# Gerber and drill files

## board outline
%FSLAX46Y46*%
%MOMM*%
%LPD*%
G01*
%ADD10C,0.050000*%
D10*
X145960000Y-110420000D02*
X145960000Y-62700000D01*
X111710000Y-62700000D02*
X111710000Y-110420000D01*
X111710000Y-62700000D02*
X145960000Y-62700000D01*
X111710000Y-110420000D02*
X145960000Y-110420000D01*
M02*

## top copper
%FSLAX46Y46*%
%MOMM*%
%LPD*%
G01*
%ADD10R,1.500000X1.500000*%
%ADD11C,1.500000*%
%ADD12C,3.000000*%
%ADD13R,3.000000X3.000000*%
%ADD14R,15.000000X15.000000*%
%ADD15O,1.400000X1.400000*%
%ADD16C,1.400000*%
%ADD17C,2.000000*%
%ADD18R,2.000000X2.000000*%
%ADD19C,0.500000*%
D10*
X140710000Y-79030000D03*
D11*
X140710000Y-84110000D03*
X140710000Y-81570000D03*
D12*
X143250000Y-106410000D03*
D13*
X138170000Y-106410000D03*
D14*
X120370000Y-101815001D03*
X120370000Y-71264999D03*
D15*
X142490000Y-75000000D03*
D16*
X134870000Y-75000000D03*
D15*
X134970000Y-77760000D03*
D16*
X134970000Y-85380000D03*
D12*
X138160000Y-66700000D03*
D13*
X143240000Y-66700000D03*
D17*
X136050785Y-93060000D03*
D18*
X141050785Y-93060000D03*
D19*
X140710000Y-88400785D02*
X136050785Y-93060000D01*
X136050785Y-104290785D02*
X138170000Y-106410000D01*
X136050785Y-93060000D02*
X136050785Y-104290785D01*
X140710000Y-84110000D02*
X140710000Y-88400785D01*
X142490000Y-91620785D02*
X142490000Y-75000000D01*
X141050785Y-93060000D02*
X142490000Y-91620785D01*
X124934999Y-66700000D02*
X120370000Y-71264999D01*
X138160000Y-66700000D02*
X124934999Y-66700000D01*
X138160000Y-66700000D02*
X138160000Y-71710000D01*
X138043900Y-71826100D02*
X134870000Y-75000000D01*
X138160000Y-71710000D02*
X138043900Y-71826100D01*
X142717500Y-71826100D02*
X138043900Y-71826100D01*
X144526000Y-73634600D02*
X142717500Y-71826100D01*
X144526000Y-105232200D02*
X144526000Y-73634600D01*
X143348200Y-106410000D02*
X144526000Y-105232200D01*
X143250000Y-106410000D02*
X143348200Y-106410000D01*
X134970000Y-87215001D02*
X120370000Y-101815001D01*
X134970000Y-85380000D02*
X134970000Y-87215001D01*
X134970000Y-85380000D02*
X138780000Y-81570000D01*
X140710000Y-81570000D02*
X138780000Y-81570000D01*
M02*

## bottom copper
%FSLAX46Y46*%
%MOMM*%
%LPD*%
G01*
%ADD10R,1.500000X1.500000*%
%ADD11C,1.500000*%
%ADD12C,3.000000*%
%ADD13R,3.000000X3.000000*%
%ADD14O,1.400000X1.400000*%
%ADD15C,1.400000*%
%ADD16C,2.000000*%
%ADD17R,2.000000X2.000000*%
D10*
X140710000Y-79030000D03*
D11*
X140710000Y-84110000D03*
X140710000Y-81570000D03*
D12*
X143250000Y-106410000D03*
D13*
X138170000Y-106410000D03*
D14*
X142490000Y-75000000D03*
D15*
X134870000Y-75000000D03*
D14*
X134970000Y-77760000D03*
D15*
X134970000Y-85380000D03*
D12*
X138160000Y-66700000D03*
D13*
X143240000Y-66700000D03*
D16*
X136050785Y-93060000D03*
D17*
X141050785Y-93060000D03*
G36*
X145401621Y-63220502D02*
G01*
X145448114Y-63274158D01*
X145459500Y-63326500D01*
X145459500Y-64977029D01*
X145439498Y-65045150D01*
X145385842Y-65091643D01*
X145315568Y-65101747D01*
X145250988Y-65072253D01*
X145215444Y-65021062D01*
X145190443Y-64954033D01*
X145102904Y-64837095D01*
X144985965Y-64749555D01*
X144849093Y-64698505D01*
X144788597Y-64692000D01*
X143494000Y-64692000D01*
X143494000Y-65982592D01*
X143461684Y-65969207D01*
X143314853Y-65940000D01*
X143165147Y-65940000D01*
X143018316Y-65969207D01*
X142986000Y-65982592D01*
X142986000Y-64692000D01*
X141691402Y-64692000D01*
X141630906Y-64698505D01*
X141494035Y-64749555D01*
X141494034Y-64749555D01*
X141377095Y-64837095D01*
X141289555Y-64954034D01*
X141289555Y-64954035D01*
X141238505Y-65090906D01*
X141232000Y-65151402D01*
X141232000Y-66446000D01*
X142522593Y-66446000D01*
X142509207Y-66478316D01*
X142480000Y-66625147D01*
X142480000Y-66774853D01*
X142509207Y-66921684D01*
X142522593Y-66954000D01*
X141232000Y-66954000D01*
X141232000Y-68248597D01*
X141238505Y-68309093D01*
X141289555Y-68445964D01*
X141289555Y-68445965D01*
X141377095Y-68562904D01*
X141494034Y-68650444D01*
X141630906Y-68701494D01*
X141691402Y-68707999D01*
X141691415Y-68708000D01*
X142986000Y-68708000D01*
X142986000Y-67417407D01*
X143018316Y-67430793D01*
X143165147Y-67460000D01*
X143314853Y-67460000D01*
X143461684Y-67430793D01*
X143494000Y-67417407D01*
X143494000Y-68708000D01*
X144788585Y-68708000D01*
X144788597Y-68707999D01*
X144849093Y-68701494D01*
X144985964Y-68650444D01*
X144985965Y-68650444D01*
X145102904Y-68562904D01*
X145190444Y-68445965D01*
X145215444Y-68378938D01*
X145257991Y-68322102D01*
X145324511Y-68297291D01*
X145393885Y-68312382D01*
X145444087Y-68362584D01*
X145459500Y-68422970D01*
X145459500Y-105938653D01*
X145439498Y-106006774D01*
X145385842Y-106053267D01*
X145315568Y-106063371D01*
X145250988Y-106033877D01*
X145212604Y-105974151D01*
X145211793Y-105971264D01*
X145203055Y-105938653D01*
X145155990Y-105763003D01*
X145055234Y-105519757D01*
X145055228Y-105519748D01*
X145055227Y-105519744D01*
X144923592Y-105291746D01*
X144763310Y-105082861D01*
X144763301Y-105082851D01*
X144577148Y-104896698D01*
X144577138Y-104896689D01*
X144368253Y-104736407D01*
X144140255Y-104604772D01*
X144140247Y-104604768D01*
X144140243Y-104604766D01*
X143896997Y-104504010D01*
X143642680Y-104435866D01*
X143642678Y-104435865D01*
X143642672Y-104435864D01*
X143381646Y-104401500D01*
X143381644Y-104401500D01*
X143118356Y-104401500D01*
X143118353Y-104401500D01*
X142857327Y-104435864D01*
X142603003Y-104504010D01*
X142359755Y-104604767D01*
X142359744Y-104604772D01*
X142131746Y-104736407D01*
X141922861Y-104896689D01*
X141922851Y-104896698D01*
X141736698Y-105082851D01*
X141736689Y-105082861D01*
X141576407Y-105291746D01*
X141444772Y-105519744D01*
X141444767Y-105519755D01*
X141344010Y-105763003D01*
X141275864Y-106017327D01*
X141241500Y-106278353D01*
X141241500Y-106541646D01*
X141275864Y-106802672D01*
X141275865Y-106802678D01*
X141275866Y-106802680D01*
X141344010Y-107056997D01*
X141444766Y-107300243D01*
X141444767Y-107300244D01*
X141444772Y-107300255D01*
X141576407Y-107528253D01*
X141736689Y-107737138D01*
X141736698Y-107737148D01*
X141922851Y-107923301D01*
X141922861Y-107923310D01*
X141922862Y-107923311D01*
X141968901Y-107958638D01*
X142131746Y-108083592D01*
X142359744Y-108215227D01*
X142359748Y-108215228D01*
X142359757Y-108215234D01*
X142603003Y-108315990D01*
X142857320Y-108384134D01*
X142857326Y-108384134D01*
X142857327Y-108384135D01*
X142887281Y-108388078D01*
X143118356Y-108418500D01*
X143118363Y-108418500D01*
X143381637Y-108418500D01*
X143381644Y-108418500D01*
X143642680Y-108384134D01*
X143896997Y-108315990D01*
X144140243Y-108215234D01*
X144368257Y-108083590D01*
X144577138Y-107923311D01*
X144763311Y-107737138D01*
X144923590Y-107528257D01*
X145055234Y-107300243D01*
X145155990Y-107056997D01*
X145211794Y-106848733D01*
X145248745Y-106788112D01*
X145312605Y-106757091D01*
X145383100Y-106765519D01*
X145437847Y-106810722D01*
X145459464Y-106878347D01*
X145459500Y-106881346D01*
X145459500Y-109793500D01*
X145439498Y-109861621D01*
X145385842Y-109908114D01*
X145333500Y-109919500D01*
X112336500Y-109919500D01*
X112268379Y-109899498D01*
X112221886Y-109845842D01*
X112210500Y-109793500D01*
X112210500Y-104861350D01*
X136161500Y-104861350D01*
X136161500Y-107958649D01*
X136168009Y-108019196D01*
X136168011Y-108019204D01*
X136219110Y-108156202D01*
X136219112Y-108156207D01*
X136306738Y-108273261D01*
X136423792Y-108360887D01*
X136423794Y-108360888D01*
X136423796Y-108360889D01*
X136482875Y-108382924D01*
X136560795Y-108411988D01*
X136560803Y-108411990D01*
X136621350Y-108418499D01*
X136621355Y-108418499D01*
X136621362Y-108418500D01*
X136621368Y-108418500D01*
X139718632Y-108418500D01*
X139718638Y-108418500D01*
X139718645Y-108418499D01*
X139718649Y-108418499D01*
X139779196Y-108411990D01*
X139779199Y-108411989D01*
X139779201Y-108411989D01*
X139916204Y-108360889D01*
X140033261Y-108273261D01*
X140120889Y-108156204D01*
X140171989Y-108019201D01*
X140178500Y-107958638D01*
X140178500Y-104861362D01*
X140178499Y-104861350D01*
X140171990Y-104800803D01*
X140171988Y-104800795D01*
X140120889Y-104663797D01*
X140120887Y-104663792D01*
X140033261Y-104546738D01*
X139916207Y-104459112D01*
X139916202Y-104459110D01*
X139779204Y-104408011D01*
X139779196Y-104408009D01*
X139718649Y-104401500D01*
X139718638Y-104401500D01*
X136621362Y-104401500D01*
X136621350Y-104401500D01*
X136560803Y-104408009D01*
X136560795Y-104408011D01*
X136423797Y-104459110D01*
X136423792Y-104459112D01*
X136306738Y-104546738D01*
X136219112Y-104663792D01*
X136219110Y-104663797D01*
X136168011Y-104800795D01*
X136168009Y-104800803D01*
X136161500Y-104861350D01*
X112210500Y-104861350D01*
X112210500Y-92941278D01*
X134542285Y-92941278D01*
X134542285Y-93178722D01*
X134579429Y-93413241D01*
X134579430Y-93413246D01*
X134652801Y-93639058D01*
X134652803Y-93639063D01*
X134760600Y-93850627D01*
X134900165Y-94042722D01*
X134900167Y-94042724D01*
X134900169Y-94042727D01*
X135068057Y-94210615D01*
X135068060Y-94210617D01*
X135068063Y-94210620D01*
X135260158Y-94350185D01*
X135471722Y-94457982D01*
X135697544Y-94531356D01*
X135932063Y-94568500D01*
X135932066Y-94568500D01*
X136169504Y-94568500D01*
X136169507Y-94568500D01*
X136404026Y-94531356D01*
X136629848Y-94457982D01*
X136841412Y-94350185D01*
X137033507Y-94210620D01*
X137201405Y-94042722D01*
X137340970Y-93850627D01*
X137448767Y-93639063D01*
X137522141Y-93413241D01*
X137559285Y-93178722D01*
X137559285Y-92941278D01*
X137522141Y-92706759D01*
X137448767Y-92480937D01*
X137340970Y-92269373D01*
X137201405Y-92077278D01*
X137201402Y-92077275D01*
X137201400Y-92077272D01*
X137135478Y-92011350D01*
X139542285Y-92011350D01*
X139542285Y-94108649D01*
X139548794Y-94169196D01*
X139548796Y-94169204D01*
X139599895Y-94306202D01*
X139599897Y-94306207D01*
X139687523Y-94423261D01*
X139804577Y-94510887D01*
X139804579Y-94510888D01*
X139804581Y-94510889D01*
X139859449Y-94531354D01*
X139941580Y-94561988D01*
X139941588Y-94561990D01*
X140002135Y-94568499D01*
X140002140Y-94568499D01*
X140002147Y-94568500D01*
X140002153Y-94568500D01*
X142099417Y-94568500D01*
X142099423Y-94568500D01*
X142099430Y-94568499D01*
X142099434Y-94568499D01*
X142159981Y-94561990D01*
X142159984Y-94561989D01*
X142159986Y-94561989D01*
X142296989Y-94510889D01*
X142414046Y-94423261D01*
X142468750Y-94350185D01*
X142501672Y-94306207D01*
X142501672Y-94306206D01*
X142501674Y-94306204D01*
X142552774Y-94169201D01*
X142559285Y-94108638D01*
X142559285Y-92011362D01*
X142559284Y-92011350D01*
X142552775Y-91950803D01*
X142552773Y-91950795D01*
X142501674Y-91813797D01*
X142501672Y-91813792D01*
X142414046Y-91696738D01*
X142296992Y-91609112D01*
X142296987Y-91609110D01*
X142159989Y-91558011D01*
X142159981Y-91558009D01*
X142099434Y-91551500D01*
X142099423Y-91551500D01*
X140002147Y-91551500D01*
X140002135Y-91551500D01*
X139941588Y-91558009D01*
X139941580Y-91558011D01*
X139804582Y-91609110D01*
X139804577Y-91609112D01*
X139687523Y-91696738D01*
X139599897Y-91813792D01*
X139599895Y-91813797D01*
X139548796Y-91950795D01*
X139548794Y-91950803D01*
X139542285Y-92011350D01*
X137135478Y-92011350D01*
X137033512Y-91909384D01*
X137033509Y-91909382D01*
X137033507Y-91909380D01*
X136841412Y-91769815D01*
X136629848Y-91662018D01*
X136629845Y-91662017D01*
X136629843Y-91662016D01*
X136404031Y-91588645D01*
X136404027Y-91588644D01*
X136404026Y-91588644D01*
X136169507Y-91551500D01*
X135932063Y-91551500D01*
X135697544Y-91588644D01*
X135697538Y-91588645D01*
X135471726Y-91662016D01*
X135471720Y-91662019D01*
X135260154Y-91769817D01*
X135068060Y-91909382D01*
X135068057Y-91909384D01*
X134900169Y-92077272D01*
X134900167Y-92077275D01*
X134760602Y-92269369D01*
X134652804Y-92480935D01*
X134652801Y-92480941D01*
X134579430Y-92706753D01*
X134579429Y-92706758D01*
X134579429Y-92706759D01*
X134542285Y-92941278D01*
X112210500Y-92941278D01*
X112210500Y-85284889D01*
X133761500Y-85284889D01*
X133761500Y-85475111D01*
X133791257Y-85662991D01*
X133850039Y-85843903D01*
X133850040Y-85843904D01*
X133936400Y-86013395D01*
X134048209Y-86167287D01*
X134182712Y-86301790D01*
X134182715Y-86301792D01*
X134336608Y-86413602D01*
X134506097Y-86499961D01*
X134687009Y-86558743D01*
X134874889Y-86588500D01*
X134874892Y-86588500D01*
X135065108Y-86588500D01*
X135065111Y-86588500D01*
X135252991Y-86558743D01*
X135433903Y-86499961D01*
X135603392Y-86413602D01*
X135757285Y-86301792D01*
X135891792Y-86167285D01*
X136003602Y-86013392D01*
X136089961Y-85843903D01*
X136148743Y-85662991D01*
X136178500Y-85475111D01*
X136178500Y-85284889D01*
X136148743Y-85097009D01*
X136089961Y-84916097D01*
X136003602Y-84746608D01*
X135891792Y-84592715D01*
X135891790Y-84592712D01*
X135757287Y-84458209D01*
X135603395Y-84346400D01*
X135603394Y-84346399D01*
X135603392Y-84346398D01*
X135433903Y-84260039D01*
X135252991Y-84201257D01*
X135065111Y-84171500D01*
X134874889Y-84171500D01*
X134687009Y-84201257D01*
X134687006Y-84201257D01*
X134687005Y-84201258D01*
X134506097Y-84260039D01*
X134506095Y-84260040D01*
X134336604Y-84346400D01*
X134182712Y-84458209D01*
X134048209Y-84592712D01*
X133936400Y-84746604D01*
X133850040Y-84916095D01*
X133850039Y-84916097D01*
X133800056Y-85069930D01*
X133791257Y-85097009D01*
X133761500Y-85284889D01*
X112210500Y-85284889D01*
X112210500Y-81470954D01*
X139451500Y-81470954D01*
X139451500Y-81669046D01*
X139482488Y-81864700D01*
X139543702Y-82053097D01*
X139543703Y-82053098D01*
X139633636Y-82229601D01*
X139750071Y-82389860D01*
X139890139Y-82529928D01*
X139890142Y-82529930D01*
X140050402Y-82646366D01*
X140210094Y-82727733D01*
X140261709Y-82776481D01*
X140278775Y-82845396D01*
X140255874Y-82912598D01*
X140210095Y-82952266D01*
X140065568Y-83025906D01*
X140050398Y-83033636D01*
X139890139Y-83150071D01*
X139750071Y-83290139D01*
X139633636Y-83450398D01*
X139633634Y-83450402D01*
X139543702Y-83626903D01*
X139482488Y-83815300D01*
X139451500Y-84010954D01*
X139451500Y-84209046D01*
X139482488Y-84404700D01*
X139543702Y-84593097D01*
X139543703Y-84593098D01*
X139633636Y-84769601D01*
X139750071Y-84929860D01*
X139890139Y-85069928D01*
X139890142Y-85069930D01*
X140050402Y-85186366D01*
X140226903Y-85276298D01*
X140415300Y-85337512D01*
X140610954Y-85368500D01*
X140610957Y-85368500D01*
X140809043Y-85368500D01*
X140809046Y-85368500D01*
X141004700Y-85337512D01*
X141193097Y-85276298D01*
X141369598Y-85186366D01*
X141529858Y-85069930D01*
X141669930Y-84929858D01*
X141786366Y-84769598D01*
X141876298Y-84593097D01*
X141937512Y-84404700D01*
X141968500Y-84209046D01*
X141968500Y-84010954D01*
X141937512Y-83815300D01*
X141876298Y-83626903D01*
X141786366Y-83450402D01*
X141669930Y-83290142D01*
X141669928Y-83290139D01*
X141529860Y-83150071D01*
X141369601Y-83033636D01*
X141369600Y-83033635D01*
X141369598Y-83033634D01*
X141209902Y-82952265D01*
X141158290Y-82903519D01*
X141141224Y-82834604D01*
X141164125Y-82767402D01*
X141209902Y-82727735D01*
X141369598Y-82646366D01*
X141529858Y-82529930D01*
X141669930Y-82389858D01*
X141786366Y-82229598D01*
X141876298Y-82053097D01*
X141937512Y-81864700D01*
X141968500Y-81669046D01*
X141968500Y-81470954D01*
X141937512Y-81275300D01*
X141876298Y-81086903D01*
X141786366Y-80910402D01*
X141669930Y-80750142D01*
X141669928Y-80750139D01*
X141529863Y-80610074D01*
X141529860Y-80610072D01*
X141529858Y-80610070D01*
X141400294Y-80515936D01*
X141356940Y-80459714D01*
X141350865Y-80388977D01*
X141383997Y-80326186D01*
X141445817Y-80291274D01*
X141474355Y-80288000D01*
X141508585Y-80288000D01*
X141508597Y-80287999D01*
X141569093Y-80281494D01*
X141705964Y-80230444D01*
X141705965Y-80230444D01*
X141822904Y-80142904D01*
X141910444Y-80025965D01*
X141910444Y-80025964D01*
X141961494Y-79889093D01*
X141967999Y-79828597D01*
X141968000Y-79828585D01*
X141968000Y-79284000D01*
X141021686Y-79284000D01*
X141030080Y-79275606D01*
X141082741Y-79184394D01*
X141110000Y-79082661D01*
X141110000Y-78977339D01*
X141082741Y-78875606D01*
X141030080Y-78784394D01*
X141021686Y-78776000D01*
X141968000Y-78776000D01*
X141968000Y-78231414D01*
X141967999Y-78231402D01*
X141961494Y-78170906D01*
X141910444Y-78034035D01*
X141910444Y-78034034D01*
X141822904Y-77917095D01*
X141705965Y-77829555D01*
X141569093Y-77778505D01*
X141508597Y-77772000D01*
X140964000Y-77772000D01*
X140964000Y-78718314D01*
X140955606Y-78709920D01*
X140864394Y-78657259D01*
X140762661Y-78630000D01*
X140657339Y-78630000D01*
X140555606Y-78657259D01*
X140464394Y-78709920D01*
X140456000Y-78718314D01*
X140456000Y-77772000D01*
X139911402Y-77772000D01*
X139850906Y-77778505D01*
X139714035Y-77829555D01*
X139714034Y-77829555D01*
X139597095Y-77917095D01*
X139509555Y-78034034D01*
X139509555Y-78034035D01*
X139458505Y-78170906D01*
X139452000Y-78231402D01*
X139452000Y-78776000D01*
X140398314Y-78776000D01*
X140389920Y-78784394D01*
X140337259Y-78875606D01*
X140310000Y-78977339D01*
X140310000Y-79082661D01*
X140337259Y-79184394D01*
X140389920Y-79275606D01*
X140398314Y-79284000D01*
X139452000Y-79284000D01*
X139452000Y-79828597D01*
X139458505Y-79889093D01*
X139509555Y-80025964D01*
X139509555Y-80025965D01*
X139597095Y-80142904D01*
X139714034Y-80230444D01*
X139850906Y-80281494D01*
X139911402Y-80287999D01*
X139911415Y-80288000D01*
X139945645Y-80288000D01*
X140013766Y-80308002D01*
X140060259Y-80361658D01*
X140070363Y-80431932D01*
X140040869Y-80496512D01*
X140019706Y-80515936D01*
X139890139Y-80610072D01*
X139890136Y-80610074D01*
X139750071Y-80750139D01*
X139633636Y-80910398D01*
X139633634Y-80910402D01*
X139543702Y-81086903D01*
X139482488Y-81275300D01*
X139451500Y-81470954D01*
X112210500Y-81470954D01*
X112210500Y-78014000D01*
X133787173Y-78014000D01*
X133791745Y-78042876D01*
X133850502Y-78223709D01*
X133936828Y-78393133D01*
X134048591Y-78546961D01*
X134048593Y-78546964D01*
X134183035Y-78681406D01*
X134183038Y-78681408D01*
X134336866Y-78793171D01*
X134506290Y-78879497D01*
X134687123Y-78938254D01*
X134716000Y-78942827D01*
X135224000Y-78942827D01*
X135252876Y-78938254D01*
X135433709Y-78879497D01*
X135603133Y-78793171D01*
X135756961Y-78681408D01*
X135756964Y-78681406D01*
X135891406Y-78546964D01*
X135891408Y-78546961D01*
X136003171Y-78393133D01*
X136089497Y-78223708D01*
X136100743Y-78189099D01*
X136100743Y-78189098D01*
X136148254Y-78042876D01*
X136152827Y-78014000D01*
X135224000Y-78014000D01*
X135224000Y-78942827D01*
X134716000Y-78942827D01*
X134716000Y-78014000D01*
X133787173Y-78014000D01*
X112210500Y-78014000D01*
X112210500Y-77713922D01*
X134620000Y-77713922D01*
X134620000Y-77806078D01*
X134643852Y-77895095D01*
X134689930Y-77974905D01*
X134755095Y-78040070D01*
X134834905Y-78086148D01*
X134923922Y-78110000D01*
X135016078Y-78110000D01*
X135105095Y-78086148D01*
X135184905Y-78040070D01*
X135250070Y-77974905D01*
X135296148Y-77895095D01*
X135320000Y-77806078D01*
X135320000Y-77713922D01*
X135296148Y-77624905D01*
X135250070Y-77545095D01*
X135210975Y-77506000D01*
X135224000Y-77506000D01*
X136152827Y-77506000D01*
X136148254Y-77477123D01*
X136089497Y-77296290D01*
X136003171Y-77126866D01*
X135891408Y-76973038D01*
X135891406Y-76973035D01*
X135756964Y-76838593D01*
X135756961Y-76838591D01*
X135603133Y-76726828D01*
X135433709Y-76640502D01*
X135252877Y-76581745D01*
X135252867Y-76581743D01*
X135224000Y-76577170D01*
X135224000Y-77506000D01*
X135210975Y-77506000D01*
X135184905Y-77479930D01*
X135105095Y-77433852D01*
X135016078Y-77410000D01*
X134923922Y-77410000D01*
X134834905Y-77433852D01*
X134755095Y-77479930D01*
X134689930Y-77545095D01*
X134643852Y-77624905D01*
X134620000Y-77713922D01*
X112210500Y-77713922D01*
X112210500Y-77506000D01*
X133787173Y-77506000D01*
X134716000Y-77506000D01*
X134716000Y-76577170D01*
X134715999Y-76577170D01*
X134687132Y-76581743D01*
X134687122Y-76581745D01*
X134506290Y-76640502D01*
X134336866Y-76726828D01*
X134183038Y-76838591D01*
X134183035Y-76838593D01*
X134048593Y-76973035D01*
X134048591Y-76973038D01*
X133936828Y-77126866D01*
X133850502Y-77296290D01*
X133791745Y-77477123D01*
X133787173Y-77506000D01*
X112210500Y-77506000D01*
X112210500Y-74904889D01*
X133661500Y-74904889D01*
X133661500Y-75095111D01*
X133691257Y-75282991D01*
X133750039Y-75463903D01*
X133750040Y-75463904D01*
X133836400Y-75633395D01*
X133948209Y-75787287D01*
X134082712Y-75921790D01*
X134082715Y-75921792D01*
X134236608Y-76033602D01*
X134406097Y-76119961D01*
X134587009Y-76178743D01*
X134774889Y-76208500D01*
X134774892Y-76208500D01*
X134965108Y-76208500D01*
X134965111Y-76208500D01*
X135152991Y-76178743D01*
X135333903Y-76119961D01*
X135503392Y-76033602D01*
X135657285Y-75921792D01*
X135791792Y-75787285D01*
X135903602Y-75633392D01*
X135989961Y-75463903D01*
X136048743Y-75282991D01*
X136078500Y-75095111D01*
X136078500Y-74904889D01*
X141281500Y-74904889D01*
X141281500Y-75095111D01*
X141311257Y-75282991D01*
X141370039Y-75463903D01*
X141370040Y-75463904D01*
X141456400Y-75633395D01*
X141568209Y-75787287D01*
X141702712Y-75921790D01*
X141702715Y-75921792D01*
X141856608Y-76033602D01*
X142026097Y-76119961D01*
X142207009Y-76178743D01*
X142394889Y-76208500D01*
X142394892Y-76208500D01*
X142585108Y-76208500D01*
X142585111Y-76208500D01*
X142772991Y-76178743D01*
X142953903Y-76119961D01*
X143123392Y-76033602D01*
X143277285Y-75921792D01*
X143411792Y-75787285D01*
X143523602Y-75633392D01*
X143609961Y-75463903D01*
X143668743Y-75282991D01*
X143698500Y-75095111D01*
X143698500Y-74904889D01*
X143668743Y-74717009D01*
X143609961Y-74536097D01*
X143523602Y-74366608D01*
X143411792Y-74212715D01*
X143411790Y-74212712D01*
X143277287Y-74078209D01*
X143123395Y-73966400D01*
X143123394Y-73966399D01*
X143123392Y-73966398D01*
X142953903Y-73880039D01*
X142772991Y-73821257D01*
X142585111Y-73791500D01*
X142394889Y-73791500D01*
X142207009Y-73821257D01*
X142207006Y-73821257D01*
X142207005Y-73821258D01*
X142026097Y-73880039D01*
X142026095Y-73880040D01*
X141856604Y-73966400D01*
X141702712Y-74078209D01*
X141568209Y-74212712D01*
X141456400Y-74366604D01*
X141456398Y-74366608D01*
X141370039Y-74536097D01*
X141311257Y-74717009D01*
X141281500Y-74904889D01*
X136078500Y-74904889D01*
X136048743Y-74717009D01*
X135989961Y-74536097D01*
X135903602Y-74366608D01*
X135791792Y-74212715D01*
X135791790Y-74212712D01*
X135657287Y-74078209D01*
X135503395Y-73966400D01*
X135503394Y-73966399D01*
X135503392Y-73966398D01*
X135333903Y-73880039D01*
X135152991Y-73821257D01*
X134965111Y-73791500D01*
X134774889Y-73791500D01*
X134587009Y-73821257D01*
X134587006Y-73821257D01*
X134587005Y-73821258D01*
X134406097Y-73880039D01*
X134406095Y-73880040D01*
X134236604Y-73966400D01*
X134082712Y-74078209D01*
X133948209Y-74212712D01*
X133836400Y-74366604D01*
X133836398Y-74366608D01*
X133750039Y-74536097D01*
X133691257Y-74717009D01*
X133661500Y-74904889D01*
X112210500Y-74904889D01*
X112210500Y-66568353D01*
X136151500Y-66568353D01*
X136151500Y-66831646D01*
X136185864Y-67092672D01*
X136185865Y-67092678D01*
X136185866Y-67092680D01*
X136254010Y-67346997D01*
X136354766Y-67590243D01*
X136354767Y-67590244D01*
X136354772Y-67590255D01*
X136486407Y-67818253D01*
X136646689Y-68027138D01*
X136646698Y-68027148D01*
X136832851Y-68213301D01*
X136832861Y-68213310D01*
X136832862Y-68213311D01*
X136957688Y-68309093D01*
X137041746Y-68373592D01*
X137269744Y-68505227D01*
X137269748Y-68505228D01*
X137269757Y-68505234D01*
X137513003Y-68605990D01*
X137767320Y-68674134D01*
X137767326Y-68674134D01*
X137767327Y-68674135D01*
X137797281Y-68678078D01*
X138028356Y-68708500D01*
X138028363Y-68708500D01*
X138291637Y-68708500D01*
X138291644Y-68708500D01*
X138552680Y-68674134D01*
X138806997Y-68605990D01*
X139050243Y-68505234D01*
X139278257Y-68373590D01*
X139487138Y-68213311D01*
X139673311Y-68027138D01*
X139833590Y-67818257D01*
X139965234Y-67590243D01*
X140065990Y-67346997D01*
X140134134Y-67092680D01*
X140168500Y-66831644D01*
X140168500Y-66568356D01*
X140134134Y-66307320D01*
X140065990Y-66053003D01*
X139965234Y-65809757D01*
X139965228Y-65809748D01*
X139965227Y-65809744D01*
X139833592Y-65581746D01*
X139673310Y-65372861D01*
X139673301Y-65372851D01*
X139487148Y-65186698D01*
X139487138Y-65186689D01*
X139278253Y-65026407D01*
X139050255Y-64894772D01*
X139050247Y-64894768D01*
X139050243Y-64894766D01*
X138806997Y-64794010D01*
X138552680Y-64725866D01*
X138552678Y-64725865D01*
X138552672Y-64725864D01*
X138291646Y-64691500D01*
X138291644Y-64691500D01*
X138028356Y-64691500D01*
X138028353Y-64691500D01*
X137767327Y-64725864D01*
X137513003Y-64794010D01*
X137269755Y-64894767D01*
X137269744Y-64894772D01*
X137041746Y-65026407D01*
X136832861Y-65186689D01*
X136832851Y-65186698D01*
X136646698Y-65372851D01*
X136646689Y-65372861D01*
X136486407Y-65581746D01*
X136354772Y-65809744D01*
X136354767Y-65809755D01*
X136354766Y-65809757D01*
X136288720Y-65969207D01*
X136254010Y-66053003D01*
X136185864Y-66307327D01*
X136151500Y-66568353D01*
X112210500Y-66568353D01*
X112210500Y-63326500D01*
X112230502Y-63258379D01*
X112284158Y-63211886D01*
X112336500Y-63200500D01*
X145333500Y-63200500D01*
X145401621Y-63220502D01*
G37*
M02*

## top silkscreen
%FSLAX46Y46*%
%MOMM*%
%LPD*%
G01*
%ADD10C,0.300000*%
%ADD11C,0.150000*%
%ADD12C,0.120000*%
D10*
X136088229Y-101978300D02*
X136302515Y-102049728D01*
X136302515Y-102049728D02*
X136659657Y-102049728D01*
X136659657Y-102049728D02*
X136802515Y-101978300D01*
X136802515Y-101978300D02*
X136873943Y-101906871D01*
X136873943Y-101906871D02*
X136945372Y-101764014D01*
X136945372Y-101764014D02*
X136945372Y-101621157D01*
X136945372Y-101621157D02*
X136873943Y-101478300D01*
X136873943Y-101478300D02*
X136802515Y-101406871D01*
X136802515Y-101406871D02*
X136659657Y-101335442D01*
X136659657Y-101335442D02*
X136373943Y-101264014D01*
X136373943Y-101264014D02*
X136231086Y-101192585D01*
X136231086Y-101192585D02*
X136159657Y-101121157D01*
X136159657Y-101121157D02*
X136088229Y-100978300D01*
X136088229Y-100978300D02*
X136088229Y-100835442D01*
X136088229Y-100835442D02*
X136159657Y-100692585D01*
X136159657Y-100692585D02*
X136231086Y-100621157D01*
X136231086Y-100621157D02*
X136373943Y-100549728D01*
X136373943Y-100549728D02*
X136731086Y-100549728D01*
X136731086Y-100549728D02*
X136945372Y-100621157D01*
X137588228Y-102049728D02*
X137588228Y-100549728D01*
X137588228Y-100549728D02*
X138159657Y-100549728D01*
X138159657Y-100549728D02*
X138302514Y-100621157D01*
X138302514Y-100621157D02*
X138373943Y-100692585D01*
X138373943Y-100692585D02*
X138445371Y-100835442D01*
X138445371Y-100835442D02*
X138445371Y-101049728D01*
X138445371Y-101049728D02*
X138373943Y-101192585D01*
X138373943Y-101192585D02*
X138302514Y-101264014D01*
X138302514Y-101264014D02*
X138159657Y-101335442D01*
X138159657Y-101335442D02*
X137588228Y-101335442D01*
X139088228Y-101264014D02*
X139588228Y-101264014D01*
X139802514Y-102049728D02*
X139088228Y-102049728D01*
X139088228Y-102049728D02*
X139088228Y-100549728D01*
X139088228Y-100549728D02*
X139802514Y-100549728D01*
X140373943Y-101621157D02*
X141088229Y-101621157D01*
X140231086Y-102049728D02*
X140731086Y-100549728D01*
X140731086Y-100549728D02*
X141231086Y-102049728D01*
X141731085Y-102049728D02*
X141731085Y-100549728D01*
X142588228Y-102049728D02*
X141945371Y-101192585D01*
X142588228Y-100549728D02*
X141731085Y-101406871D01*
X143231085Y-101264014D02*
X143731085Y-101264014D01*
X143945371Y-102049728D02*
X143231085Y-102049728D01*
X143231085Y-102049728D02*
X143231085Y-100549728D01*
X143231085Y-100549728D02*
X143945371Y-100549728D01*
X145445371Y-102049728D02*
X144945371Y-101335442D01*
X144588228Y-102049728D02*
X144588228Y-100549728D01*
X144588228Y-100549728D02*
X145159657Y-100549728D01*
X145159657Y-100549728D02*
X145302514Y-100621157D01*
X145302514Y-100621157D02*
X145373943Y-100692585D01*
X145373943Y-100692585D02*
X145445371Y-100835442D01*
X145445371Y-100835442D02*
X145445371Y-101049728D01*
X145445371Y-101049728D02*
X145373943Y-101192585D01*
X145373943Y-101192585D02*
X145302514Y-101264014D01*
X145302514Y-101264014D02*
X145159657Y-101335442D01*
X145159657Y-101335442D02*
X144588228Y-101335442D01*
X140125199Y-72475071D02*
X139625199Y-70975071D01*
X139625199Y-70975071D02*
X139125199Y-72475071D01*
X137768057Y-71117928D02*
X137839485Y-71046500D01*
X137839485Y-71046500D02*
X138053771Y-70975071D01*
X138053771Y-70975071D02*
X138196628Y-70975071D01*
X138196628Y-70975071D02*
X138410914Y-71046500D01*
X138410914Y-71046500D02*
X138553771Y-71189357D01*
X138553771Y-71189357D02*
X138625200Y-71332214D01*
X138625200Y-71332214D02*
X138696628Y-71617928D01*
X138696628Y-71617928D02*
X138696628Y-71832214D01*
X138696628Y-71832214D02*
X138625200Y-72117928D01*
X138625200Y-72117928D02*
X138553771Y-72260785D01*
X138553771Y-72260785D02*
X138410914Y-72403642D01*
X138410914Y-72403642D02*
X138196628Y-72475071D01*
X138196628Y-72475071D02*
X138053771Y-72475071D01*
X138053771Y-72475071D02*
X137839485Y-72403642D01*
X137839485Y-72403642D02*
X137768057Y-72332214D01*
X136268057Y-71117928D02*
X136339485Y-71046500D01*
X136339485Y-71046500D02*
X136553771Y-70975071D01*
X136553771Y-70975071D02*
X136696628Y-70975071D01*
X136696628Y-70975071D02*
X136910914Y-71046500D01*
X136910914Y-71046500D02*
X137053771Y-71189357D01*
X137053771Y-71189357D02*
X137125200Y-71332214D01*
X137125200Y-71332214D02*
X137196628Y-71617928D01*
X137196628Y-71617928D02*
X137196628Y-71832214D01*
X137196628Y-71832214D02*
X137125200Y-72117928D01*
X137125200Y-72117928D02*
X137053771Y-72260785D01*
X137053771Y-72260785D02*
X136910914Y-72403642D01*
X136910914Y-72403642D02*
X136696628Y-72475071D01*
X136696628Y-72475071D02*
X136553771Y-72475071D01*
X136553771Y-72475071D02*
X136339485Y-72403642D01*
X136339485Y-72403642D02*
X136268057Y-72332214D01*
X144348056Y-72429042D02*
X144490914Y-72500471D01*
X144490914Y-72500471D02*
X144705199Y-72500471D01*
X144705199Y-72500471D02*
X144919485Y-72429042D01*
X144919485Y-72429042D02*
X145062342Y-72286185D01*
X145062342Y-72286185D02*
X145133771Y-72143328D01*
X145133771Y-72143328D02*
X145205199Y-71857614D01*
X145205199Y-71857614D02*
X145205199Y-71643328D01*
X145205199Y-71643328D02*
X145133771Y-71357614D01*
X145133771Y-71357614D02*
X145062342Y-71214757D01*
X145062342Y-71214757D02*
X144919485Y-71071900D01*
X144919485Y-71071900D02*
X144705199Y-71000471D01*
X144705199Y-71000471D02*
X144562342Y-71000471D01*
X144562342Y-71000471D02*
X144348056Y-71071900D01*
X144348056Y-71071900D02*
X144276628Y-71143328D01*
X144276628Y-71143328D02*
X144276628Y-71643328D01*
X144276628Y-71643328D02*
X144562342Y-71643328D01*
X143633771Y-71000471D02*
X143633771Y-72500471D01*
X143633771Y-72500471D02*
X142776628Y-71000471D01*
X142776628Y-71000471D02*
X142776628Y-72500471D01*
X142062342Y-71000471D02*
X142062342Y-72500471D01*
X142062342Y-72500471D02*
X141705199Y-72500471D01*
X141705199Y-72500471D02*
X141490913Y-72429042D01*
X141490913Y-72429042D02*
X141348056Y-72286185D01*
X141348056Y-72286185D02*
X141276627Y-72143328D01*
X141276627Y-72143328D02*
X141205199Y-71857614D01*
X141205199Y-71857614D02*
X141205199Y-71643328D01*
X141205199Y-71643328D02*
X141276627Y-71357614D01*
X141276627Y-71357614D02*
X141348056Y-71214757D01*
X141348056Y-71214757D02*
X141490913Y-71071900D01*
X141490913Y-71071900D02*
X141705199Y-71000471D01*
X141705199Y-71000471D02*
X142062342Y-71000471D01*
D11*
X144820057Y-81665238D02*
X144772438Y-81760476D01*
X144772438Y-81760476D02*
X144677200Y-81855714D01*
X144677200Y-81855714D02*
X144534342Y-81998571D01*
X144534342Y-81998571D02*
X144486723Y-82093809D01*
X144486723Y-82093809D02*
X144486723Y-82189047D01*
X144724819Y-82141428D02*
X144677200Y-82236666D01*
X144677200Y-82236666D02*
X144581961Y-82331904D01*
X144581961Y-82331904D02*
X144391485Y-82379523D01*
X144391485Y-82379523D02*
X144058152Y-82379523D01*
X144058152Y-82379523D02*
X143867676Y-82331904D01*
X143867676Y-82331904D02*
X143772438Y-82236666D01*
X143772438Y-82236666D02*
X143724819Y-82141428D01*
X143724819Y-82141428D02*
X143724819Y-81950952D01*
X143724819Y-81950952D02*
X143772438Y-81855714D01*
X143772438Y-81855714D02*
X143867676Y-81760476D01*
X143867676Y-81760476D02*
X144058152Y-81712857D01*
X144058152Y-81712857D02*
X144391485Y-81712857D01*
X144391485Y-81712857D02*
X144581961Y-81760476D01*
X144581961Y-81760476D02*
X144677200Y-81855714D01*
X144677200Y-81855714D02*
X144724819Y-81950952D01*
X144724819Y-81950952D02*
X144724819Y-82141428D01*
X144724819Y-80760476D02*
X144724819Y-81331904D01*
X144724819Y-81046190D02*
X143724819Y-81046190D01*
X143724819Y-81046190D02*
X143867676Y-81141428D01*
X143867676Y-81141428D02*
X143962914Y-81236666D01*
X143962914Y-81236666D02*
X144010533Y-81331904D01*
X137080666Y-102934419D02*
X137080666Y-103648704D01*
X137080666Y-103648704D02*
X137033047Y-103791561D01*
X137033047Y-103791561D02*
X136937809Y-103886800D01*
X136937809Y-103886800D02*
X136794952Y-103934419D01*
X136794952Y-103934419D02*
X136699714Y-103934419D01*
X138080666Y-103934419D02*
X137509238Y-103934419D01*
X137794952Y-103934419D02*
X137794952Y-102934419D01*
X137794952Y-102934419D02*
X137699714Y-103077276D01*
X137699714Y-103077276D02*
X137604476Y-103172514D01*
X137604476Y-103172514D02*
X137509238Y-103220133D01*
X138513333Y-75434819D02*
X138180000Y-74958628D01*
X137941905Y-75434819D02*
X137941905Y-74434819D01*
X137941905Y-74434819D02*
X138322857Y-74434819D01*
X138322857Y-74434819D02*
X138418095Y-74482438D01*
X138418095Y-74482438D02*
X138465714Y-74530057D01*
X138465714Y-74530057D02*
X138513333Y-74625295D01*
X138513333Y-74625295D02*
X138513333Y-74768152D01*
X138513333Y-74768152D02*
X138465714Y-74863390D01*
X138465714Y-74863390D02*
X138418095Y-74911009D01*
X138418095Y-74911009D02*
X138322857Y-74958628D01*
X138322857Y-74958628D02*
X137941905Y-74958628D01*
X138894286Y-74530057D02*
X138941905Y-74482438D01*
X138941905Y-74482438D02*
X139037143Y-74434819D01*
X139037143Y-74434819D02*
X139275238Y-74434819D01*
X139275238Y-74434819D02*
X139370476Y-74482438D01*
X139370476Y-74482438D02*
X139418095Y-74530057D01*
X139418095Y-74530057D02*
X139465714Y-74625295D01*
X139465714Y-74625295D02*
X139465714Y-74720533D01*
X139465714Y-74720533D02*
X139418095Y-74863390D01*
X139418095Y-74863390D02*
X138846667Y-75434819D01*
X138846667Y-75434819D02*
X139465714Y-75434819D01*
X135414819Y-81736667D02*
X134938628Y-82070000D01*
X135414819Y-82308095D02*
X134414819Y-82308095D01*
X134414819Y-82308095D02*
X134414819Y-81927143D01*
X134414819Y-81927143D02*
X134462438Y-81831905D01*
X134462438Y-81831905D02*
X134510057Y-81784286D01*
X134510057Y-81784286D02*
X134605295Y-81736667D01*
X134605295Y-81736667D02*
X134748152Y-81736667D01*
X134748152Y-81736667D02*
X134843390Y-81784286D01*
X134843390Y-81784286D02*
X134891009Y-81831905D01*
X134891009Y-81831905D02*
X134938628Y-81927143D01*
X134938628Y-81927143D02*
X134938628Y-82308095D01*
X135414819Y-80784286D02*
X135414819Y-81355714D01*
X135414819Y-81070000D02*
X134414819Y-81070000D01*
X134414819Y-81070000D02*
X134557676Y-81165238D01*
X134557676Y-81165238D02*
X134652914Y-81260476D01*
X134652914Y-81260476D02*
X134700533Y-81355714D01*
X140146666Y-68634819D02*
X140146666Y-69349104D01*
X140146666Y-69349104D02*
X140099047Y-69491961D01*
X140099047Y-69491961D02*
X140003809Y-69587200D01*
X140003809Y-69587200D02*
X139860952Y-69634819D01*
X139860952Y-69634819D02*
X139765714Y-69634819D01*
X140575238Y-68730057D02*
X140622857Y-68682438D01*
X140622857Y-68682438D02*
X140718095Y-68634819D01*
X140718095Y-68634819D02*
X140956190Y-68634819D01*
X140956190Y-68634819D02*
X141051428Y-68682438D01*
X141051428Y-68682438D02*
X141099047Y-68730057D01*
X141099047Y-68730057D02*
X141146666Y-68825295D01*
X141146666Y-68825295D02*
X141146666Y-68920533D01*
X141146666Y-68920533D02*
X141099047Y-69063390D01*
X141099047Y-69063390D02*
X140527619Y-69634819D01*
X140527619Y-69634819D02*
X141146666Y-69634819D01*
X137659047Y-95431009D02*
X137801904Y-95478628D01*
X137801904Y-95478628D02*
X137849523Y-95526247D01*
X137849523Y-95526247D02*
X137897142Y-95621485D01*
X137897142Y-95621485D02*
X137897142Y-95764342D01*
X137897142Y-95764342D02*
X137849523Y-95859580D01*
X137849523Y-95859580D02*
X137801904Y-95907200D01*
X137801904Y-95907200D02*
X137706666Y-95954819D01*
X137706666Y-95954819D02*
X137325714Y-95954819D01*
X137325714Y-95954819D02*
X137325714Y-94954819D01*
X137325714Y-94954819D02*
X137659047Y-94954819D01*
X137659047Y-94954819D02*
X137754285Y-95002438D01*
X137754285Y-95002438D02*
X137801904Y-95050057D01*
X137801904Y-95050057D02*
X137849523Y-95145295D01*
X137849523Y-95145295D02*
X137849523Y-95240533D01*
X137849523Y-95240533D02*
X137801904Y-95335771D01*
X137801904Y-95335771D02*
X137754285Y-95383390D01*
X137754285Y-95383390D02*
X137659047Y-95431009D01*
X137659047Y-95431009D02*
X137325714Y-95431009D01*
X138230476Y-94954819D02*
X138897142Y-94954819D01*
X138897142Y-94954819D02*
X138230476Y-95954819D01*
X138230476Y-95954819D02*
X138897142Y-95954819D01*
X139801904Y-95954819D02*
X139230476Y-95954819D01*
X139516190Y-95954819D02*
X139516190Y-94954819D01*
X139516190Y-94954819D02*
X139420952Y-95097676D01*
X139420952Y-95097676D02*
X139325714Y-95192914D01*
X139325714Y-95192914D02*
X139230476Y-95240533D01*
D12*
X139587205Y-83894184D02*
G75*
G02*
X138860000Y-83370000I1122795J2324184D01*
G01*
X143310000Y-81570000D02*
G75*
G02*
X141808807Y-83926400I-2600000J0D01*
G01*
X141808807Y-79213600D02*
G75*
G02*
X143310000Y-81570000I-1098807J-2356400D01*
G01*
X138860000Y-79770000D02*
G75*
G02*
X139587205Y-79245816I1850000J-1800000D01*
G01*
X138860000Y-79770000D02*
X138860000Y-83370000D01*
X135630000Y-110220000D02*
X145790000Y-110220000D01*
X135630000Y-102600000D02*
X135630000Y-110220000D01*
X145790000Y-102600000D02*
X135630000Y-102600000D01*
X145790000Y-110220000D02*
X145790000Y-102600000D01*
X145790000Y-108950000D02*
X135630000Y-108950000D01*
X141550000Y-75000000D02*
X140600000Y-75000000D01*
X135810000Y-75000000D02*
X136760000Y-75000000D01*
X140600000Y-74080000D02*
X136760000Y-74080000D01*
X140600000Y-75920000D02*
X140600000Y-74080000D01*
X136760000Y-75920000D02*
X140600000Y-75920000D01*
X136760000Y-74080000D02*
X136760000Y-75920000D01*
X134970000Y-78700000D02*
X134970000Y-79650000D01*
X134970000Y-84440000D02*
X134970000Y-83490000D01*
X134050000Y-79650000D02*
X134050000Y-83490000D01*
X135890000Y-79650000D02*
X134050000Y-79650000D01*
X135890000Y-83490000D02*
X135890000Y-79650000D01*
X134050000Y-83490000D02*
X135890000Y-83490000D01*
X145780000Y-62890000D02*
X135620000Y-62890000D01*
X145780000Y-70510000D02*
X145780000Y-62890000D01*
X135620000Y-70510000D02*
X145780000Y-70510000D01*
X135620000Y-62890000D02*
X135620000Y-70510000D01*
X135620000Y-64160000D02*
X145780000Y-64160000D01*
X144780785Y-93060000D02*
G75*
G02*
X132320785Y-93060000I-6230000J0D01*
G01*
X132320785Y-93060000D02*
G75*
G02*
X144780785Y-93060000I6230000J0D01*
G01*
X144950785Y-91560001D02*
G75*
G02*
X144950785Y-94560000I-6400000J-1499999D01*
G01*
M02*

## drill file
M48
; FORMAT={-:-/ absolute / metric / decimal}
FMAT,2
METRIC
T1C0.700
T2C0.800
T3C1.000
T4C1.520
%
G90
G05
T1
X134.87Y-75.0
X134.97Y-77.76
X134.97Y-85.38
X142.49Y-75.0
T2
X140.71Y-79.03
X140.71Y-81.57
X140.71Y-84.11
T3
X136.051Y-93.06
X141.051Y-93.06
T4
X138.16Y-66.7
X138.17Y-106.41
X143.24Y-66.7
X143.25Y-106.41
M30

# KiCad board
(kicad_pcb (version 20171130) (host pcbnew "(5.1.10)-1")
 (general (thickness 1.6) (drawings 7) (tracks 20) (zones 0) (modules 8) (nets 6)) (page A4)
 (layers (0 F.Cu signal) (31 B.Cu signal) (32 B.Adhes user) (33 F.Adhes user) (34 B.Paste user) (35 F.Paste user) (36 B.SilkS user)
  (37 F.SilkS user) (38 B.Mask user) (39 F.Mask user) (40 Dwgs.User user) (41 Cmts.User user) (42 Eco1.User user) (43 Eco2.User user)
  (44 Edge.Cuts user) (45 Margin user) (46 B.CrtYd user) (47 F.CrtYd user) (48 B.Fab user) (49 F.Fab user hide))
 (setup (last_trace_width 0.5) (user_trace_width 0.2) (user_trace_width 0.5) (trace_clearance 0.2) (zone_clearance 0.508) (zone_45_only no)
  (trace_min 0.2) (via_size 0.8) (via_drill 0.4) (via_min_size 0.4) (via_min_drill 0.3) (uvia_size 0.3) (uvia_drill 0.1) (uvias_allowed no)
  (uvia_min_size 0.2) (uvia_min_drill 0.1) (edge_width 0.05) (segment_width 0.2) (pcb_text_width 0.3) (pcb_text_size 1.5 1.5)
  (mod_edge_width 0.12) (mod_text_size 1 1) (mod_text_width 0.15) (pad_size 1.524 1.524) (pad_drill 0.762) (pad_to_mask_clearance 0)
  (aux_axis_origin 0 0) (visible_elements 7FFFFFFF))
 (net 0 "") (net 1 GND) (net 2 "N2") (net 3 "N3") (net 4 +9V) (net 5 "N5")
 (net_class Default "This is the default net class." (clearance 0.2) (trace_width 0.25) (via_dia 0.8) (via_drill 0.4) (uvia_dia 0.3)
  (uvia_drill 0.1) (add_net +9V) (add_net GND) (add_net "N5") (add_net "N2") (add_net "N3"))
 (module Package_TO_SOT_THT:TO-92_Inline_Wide (layer F.Cu) (at 140.71 79.03 270)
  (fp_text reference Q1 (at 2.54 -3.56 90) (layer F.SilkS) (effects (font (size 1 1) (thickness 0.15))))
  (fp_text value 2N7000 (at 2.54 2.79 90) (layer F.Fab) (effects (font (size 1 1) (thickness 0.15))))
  (fp_arc (start 2.54 0) (end 4.34 1.85) (angle -20) (layer F.SilkS) (width 0.12))
  (fp_arc (start 2.54 0) (end 2.54 -2.6) (angle 65) (layer F.SilkS) (width 0.12))
  (fp_arc (start 2.54 0) (end 2.54 -2.6) (angle -65) (layer F.SilkS) (width 0.12))
  (fp_arc (start 2.54 0) (end 0.74 1.85) (angle 20) (layer F.SilkS) (width 0.12))
  (fp_line (start 0.74 1.85) (end 4.34 1.85) (layer F.SilkS) (width 0.12))
  (pad 1 thru_hole rect (at 0 0 270) (size 1.5 1.5) (drill 0.8) (layers *.Cu *.Mask) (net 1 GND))
  (pad 3 thru_hole circle (at 5.08 0 270) (size 1.5 1.5) (drill 0.8) (layers *.Cu *.Mask) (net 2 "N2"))
  (pad 2 thru_hole circle (at 2.54 0 270) (size 1.5 1.5) (drill 0.8) (layers *.Cu *.Mask) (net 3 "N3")))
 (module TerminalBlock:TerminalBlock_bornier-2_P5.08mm (layer F.Cu) (at 138.17 106.41)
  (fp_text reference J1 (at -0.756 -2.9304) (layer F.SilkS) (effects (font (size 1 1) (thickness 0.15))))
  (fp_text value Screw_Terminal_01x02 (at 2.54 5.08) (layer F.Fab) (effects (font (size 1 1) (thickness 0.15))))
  (fp_line (start -2.54 3.81) (end 7.62 3.81) (layer F.SilkS) (width 0.12))
  (fp_line (start -2.54 -3.81) (end -2.54 3.81) (layer F.SilkS) (width 0.12))
  (fp_line (start 7.62 -3.81) (end -2.54 -3.81) (layer F.SilkS) (width 0.12))
  (fp_line (start 7.62 3.81) (end 7.62 -3.81) (layer F.SilkS) (width 0.12))
  (fp_line (start 7.62 2.54) (end -2.54 2.54) (layer F.SilkS) (width 0.12))
  (pad 2 thru_hole circle (at 5.08 0) (size 3 3) (drill 1.52) (layers *.Cu *.Mask) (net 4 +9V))
  (pad 1 thru_hole rect (at 0 0) (size 3 3) (drill 1.52) (layers *.Cu *.Mask) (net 2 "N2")))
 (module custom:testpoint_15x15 (layer F.Cu) (at 120.37 101.815001)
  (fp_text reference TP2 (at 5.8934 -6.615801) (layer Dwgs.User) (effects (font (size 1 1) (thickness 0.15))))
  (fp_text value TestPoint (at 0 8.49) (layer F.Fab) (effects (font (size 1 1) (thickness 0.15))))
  (pad 1 smd rect (at 0 0) (size 15 15) (layers F.Cu F.Paste F.Mask) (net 3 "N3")))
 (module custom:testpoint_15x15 (layer F.Cu) (at 120.37 71.264999)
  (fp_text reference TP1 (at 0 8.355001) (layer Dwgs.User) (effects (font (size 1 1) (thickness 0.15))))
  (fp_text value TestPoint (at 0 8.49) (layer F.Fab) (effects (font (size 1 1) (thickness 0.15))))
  (pad 1 smd rect (at 0 0) (size 15 15) (layers F.Cu F.Paste F.Mask) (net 4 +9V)))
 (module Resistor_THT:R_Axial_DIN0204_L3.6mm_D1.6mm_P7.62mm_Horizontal (layer F.Cu) (at 134.87 75)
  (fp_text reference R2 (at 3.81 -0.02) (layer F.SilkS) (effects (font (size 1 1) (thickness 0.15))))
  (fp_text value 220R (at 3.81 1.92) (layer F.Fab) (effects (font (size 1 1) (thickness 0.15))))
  (fp_line (start 6.68 0) (end 5.73 0) (layer F.SilkS) (width 0.12))
  (fp_line (start 0.94 0) (end 1.89 0) (layer F.SilkS) (width 0.12))
  (fp_line (start 5.73 -0.92) (end 1.89 -0.92) (layer F.SilkS) (width 0.12))
  (fp_line (start 5.73 0.92) (end 5.73 -0.92) (layer F.SilkS) (width 0.12))
  (fp_line (start 1.89 0.92) (end 5.73 0.92) (layer F.SilkS) (width 0.12))
  (fp_line (start 1.89 -0.92) (end 1.89 0.92) (layer F.SilkS) (width 0.12))
  (pad 2 thru_hole oval (at 7.62 0) (size 1.4 1.4) (drill 0.7) (layers *.Cu *.Mask) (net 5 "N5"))
  (pad 1 thru_hole circle (at 0 0) (size 1.4 1.4) (drill 0.7) (layers *.Cu *.Mask) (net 4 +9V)))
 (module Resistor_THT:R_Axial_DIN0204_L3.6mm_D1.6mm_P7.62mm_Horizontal (layer F.Cu) (at 134.97 85.38 90)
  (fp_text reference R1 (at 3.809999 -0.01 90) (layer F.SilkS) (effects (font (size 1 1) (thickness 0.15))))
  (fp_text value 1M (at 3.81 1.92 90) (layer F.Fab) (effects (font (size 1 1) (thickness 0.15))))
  (fp_line (start 6.68 0) (end 5.73 0) (layer F.SilkS) (width 0.12))
  (fp_line (start 0.94 0) (end 1.89 0) (layer F.SilkS) (width 0.12))
  (fp_line (start 5.73 -0.92) (end 1.89 -0.92) (layer F.SilkS) (width 0.12))
  (fp_line (start 5.73 0.92) (end 5.73 -0.92) (layer F.SilkS) (width 0.12))
  (fp_line (start 1.89 0.92) (end 5.73 0.92) (layer F.SilkS) (width 0.12))
  (fp_line (start 1.89 -0.92) (end 1.89 0.92) (layer F.SilkS) (width 0.12))
  (pad 2 thru_hole oval (at 7.62 0 90) (size 1.4 1.4) (drill 0.7) (layers *.Cu *.Mask) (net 1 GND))
  (pad 1 thru_hole circle (at 0 0 90) (size 1.4 1.4) (drill 0.7) (layers *.Cu *.Mask) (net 3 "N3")))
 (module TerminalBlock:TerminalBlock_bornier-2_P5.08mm (layer F.Cu) (at 143.24 66.7 180)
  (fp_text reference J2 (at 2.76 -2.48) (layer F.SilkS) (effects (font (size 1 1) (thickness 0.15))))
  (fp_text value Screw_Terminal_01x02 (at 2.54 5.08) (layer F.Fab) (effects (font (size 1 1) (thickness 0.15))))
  (fp_line (start -2.54 3.81) (end 7.62 3.81) (layer F.SilkS) (width 0.12))
  (fp_line (start -2.54 -3.81) (end -2.54 3.81) (layer F.SilkS) (width 0.12))
  (fp_line (start 7.62 -3.81) (end -2.54 -3.81) (layer F.SilkS) (width 0.12))
  (fp_line (start 7.62 3.81) (end 7.62 -3.81) (layer F.SilkS) (width 0.12))
  (fp_line (start 7.62 2.54) (end -2.54 2.54) (layer F.SilkS) (width 0.12))
  (pad 2 thru_hole circle (at 5.08 0 180) (size 3 3) (drill 1.52) (layers *.Cu *.Mask) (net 4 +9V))
  (pad 1 thru_hole rect (at 0 0 180) (size 3 3) (drill 1.52) (layers *.Cu *.Mask) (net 1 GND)))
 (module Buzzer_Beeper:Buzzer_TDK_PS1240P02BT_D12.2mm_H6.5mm (layer F.Cu) (at 141.050785 93.06 180)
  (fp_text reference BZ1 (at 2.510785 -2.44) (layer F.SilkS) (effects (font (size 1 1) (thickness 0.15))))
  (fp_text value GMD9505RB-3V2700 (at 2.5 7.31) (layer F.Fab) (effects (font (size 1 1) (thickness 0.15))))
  (fp_circle (center 2.5 0) (end 8.73 0) (layer F.SilkS) (width 0.12))
  (fp_arc (start 2.5 0) (end -3.9 -1.5) (angle -26.38121493) (layer F.SilkS) (width 0.12))
  (pad 2 thru_hole circle (at 5 0 180) (size 2 2) (drill 1) (layers *.Cu *.Mask) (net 2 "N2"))
  (pad 1 thru_hole rect (at 0 0 180) (size 2 2) (drill 1) (layers *.Cu *.Mask) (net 5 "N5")))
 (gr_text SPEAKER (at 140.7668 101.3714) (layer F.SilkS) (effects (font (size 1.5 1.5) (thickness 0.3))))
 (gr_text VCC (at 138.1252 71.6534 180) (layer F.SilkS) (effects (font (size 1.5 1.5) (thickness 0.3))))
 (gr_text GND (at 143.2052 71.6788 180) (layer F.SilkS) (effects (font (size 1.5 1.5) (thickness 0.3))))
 (gr_line (start 145.96 110.42) (end 145.96 62.7) (layer Edge.Cuts) (width 0.05))
 (gr_line (start 111.71 62.7) (end 111.71 110.42) (layer Edge.Cuts) (width 0.05))
 (gr_line (start 111.71 62.7) (end 145.96 62.7) (layer Edge.Cuts) (width 0.05))
 (gr_line (start 111.71 110.42) (end 145.96 110.42) (layer Edge.Cuts) (width 0.05))
 (segment (start 140.71 88.400785) (end 136.050785 93.06) (width 0.5) (layer F.Cu) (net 2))
 (segment (start 136.050785 104.290785) (end 138.17 106.41) (width 0.5) (layer F.Cu) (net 2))
 (segment (start 136.050785 93.06) (end 136.050785 104.290785) (width 0.5) (layer F.Cu) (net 2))
 (segment (start 140.71 84.11) (end 140.71 88.400785) (width 0.5) (layer F.Cu) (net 2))
 (segment (start 142.49 91.620785) (end 142.49 75) (width 0.5) (layer F.Cu) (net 5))
 (segment (start 141.050785 93.06) (end 142.49 91.620785) (width 0.5) (layer F.Cu) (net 5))
 (segment (start 124.934999 66.7) (end 120.37 71.264999) (width 0.5) (layer F.Cu) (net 4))
 (segment (start 138.16 66.7) (end 124.934999 66.7) (width 0.5) (layer F.Cu) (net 4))
 (segment (start 138.16 66.7) (end 138.16 71.71) (width 0.5) (layer F.Cu) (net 4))
 (segment (start 138.0439 71.8261) (end 134.87 75) (width 0.5) (layer F.Cu) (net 4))
 (segment (start 138.16 71.71) (end 138.0439 71.8261) (width 0.5) (layer F.Cu) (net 4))
 (segment (start 142.7175 71.8261) (end 138.0439 71.8261) (width 0.5) (layer F.Cu) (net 4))
 (segment (start 144.526 73.6346) (end 142.7175 71.8261) (width 0.5) (layer F.Cu) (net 4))
 (segment (start 144.526 105.2322) (end 144.526 73.6346) (width 0.5) (layer F.Cu) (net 4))
 (segment (start 143.3482 106.41) (end 144.526 105.2322) (width 0.5) (layer F.Cu) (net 4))
 (segment (start 143.25 106.41) (end 143.3482 106.41) (width 0.5) (layer F.Cu) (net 4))
 (segment (start 134.97 87.215001) (end 120.37 101.815001) (width 0.5) (layer F.Cu) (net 3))
 (segment (start 134.97 85.38) (end 134.97 87.215001) (width 0.5) (layer F.Cu) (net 3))
 (segment (start 134.97 85.38) (end 138.78 81.57) (width 0.5) (layer F.Cu) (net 3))
 (segment (start 140.71 81.57) (end 138.78 81.57) (width 0.5) (layer F.Cu) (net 3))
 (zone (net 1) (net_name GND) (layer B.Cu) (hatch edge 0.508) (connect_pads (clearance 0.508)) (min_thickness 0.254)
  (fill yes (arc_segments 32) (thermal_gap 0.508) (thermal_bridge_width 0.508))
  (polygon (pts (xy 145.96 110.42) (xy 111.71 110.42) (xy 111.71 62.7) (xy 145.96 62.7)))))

